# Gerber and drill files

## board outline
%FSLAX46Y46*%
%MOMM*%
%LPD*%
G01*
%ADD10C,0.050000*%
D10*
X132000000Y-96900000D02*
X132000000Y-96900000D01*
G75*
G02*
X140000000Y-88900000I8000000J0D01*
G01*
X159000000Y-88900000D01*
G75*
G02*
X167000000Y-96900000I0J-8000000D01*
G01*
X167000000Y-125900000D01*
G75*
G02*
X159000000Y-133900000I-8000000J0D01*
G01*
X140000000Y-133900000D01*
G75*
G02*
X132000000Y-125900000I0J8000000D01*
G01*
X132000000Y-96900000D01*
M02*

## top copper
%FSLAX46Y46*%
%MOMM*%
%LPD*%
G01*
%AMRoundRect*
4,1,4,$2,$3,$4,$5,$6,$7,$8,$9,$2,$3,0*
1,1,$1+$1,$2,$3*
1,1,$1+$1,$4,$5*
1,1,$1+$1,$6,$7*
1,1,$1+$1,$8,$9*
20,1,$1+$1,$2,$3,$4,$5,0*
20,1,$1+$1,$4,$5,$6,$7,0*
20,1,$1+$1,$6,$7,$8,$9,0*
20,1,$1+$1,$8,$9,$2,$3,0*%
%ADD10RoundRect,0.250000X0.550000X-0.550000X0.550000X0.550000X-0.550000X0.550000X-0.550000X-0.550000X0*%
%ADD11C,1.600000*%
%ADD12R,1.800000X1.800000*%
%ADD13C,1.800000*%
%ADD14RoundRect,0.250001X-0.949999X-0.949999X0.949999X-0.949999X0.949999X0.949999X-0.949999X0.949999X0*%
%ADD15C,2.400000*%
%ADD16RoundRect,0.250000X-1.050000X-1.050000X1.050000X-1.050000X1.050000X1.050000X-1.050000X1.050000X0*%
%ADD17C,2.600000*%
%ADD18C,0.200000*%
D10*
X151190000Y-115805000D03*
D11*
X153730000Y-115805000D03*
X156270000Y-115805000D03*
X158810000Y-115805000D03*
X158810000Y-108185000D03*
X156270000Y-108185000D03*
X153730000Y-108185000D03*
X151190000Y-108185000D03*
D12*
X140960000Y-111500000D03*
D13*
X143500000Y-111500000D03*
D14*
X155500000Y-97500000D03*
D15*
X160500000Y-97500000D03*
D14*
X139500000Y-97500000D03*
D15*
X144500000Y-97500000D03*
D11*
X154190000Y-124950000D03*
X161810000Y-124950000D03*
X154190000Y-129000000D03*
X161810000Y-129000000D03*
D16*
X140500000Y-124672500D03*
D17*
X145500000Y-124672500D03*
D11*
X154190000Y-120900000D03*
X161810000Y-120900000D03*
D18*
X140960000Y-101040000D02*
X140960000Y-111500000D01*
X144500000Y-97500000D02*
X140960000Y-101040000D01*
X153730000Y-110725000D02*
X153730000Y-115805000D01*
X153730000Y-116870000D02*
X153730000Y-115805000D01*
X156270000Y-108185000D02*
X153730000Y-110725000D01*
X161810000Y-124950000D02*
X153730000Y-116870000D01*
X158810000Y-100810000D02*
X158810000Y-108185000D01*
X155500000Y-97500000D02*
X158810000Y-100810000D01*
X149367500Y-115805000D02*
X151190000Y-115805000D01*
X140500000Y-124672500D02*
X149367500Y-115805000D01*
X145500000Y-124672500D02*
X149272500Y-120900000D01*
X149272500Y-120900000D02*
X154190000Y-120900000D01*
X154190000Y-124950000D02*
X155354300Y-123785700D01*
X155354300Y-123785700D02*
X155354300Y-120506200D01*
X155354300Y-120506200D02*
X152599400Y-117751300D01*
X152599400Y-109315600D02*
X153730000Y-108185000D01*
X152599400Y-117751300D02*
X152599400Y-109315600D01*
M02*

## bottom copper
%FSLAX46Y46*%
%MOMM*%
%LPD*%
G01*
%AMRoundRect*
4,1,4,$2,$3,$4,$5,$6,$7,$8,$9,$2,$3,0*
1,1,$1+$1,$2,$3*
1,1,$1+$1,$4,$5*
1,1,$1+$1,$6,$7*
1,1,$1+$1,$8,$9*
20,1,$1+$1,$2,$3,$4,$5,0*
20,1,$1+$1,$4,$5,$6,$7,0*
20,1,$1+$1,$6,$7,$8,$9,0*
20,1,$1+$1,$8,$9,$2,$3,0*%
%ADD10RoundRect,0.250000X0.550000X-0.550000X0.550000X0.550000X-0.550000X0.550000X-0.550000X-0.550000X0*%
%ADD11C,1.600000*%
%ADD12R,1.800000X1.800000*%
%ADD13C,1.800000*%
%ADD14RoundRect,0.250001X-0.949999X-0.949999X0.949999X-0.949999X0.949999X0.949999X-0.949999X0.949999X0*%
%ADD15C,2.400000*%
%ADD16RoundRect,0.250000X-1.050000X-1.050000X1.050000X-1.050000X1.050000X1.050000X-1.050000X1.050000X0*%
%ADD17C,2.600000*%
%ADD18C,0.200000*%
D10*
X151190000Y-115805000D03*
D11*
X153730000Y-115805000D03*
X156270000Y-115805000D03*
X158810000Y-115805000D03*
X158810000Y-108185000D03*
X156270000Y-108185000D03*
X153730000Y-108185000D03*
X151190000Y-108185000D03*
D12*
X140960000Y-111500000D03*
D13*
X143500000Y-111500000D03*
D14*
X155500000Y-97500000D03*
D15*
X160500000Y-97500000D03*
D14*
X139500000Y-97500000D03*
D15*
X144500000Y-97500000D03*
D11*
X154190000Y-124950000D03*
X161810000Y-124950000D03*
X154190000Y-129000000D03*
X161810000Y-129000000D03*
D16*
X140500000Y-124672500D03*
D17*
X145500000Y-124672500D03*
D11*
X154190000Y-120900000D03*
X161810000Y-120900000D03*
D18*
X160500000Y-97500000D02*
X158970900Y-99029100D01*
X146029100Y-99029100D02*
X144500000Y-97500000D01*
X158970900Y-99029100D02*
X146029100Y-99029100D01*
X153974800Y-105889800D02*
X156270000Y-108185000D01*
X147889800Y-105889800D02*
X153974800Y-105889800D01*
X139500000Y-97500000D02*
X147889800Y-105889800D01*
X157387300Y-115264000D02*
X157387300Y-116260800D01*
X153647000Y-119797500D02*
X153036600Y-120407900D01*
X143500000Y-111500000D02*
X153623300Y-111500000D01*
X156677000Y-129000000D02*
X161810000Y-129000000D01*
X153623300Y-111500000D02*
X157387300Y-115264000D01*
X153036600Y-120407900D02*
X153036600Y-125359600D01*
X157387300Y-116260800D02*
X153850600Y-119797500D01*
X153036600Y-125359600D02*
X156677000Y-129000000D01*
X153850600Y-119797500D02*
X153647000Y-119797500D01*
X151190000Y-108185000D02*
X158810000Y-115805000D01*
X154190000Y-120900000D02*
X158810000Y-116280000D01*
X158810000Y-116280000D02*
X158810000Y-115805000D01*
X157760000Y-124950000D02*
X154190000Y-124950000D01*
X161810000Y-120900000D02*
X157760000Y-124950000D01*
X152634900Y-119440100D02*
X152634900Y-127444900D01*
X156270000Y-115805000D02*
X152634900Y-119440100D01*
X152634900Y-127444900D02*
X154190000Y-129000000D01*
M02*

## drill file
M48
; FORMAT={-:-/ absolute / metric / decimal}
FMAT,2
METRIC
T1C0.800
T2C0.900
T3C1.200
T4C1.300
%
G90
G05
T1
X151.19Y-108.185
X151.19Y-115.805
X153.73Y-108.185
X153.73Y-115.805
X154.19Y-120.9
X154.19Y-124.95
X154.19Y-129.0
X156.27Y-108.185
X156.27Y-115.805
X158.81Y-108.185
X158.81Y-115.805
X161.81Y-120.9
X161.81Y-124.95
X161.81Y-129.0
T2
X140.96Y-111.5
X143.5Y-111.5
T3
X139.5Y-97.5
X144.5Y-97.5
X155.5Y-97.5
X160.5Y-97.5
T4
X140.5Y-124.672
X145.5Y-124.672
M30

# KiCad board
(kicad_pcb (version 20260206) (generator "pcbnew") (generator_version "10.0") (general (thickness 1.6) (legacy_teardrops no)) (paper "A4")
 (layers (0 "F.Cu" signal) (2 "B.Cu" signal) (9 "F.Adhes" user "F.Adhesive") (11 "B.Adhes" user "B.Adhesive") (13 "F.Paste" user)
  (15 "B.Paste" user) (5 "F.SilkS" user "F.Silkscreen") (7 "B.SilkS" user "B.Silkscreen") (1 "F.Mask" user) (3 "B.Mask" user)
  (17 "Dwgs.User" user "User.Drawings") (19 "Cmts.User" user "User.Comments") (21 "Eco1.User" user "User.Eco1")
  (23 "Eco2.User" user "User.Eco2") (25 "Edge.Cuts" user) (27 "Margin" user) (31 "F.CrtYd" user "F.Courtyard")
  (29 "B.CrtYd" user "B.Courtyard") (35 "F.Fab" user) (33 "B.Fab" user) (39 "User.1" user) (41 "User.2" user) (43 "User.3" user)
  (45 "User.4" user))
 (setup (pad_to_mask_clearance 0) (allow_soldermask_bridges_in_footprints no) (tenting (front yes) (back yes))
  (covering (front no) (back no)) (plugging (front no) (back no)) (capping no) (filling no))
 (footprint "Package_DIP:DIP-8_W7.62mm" (layer "F.Cu") (at 151.19 115.805 90)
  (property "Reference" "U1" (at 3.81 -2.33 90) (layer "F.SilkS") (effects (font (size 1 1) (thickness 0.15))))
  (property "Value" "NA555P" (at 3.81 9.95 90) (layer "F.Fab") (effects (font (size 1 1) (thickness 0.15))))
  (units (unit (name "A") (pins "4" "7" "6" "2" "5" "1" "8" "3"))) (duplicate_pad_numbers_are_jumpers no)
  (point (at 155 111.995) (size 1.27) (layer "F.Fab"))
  (pad "1" thru_hole roundrect (at 0 0 90) (size 1.6 1.6) (drill 0.8) (layers "*.Cu" "*.Mask") (remove_unused_layers no)
   (roundrect_rratio 0.15625) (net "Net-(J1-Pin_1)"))
  (pad "2" thru_hole circle (at 0 2.54 90) (size 1.6 1.6) (drill 0.8) (layers "*.Cu" "*.Mask") (remove_unused_layers no)
   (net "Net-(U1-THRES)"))
  (pad "3" thru_hole circle (at 0 5.08 90) (size 1.6 1.6) (drill 0.8) (layers "*.Cu" "*.Mask") (remove_unused_layers no)
   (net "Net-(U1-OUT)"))
  (pad "4" thru_hole circle (at 0 7.62 90) (size 1.6 1.6) (drill 0.8) (layers "*.Cu" "*.Mask") (remove_unused_layers no)
   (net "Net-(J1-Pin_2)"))
  (pad "5" thru_hole circle (at 7.62 7.62 90) (size 1.6 1.6) (drill 0.8) (layers "*.Cu" "*.Mask") (remove_unused_layers no)
   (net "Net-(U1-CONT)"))
  (pad "6" thru_hole circle (at 7.62 5.08 90) (size 1.6 1.6) (drill 0.8) (layers "*.Cu" "*.Mask") (remove_unused_layers no)
   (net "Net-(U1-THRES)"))
  (pad "7" thru_hole circle (at 7.62 2.54 90) (size 1.6 1.6) (drill 0.8) (layers "*.Cu" "*.Mask") (remove_unused_layers no)
   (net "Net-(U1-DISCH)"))
  (pad "8" thru_hole circle (at 7.62 0 90) (size 1.6 1.6) (drill 0.8) (layers "*.Cu" "*.Mask") (remove_unused_layers no)
   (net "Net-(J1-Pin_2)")))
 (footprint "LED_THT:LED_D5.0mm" (layer "F.Cu") (at 140.96 111.5)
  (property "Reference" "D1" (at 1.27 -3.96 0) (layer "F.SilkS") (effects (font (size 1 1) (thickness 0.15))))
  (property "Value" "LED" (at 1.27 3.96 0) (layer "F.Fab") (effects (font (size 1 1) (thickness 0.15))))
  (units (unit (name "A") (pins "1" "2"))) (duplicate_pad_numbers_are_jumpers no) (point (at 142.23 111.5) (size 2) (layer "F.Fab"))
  (pad "1" thru_hole rect (at 0 0) (size 1.8 1.8) (drill 0.9) (layers "*.Cu" "*.Mask") (remove_unused_layers no) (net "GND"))
  (pad "2" thru_hole circle (at 2.54 0) (size 1.8 1.8) (drill 0.9) (layers "*.Cu" "*.Mask") (remove_unused_layers no) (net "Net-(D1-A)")))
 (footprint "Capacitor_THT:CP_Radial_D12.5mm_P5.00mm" (layer "F.Cu") (at 155.5 97.5)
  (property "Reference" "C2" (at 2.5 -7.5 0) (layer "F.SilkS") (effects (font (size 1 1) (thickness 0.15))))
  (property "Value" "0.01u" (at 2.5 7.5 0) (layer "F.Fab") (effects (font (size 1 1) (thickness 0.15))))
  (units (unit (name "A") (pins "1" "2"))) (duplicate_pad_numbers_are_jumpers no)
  (pad "1" thru_hole roundrect (at 0 0) (size 2.4 2.4) (drill 1.2) (layers "*.Cu" "*.Mask") (remove_unused_layers no)
   (roundrect_rratio 0.104167) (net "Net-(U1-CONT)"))
  (pad "2" thru_hole circle (at 5 0) (size 2.4 2.4) (drill 1.2) (layers "*.Cu" "*.Mask") (remove_unused_layers no) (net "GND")))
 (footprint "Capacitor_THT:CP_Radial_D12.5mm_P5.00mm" (layer "F.Cu") (at 139.5 97.5)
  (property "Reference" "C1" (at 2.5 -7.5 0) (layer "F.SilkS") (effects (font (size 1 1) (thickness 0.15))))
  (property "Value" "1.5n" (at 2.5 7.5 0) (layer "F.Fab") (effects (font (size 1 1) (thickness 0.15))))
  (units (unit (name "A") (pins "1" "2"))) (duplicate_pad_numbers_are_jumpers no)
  (pad "1" thru_hole roundrect (at 0 0) (size 2.4 2.4) (drill 1.2) (layers "*.Cu" "*.Mask") (remove_unused_layers no)
   (roundrect_rratio 0.104167) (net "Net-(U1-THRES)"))
  (pad "2" thru_hole circle (at 5 0) (size 2.4 2.4) (drill 1.2) (layers "*.Cu" "*.Mask") (remove_unused_layers no) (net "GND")))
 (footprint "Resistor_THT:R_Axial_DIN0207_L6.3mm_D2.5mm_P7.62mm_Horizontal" (layer "F.Cu") (at 154.19 124.95)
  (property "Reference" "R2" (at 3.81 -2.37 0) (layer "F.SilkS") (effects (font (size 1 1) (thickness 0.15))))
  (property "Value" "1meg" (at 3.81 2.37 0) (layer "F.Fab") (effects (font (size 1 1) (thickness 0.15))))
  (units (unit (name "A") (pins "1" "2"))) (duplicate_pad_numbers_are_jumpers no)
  (pad "1" thru_hole circle (at 0 0) (size 1.6 1.6) (drill 0.8) (layers "*.Cu" "*.Mask") (remove_unused_layers no) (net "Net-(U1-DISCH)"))
  (pad "2" thru_hole circle (at 7.62 0) (size 1.6 1.6) (drill 0.8) (layers "*.Cu" "*.Mask") (remove_unused_layers no) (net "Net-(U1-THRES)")))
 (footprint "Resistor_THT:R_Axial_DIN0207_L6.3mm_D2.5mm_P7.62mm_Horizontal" (layer "F.Cu") (at 154.19 129)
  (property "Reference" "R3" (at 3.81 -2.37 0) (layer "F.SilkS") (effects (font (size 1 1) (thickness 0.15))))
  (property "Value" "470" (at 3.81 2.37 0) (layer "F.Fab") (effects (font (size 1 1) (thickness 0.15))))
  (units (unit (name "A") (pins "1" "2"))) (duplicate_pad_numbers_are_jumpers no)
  (pad "1" thru_hole circle (at 0 0) (size 1.6 1.6) (drill 0.8) (layers "*.Cu" "*.Mask") (remove_unused_layers no) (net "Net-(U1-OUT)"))
  (pad "2" thru_hole circle (at 7.62 0) (size 1.6 1.6) (drill 0.8) (layers "*.Cu" "*.Mask") (remove_unused_layers no) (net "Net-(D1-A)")))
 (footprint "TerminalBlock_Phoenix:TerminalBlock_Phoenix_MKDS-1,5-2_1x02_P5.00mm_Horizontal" (layer "F.Cu") (at 140.5 124.6725)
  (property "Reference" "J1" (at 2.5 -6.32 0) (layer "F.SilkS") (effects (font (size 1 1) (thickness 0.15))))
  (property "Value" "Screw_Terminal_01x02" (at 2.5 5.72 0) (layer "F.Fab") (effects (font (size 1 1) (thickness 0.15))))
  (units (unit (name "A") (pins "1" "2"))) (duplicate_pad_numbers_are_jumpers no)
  (pad "1" thru_hole roundrect (at 0 0) (size 2.6 2.6) (drill 1.3) (layers "*.Cu" "*.Mask") (remove_unused_layers no)
   (roundrect_rratio 0.096154) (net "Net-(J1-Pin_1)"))
  (pad "2" thru_hole circle (at 5 0) (size 2.6 2.6) (drill 1.3) (layers "*.Cu" "*.Mask") (remove_unused_layers no) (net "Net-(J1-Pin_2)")))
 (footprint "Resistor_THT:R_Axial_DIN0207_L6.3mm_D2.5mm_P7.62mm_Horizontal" (layer "F.Cu") (at 154.19 120.9)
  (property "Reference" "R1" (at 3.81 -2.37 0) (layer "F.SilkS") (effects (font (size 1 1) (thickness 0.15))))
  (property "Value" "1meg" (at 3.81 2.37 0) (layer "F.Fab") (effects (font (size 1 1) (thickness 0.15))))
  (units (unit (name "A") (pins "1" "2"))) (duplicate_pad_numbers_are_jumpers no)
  (pad "1" thru_hole circle (at 0 0) (size 1.6 1.6) (drill 0.8) (layers "*.Cu" "*.Mask") (remove_unused_layers no) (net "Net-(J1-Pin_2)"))
  (pad "2" thru_hole circle (at 7.62 0) (size 1.6 1.6) (drill 0.8) (layers "*.Cu" "*.Mask") (remove_unused_layers no) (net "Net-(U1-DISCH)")))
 (gr_rect (start 132 88.9) (end 167 133.9) (radius 8) (stroke (width 0.05) (type solid)) (fill no) (layer "Edge.Cuts"))
 (segment (start 140.96 101.04) (end 140.96 111.5) (width 0.2) (layer "F.Cu") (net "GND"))
 (segment (start 144.5 97.5) (end 140.96 101.04) (width 0.2) (layer "F.Cu") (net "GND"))
 (segment (start 160.5 97.5) (end 158.9709 99.0291) (width 0.2) (layer "B.Cu") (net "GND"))
 (segment (start 146.0291 99.0291) (end 144.5 97.5) (width 0.2) (layer "B.Cu") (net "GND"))
 (segment (start 158.9709 99.0291) (end 146.0291 99.0291) (width 0.2) (layer "B.Cu") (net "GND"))
 (segment (start 153.73 110.725) (end 153.73 115.805) (width 0.2) (layer "F.Cu") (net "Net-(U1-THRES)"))
 (segment (start 153.73 116.87) (end 153.73 115.805) (width 0.2) (layer "F.Cu") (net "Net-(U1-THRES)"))
 (segment (start 156.27 108.185) (end 153.73 110.725) (width 0.2) (layer "F.Cu") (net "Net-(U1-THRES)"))
 (segment (start 161.81 124.95) (end 153.73 116.87) (width 0.2) (layer "F.Cu") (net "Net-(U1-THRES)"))
 (segment (start 153.9748 105.8898) (end 156.27 108.185) (width 0.2) (layer "B.Cu") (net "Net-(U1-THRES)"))
 (segment (start 147.8898 105.8898) (end 153.9748 105.8898) (width 0.2) (layer "B.Cu") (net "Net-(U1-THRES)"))
 (segment (start 139.5 97.5) (end 147.8898 105.8898) (width 0.2) (layer "B.Cu") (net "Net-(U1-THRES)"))
 (segment (start 158.81 100.81) (end 158.81 108.185) (width 0.2) (layer "F.Cu") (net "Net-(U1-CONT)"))
 (segment (start 155.5 97.5) (end 158.81 100.81) (width 0.2) (layer "F.Cu") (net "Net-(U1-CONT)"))
 (segment (start 157.3873 115.264) (end 157.3873 116.2608) (width 0.2) (layer "B.Cu") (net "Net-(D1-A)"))
 (segment (start 153.647 119.7975) (end 153.0366 120.4079) (width 0.2) (layer "B.Cu") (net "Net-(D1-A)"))
 (segment (start 143.5 111.5) (end 153.6233 111.5) (width 0.2) (layer "B.Cu") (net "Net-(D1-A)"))
 (segment (start 156.677 129) (end 161.81 129) (width 0.2) (layer "B.Cu") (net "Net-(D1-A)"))
 (segment (start 153.6233 111.5) (end 157.3873 115.264) (width 0.2) (layer "B.Cu") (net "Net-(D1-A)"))
 (segment (start 153.0366 120.4079) (end 153.0366 125.3596) (width 0.2) (layer "B.Cu") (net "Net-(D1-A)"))
 (segment (start 157.3873 116.2608) (end 153.8506 119.7975) (width 0.2) (layer "B.Cu") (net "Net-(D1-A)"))
 (segment (start 153.0366 125.3596) (end 156.677 129) (width 0.2) (layer "B.Cu") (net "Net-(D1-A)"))
 (segment (start 153.8506 119.7975) (end 153.647 119.7975) (width 0.2) (layer "B.Cu") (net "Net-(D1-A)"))
 (segment (start 149.3675 115.805) (end 151.19 115.805) (width 0.2) (layer "F.Cu") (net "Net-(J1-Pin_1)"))
 (segment (start 140.5 124.6725) (end 149.3675 115.805) (width 0.2) (layer "F.Cu") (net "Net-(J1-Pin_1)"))
 (segment (start 145.5 124.6725) (end 149.2725 120.9) (width 0.2) (layer "F.Cu") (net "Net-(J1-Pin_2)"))
 (segment (start 149.2725 120.9) (end 154.19 120.9) (width 0.2) (layer "F.Cu") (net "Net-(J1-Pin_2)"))
 (segment (start 151.19 108.185) (end 158.81 115.805) (width 0.2) (layer "B.Cu") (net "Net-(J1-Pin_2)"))
 (segment (start 154.19 120.9) (end 158.81 116.28) (width 0.2) (layer "B.Cu") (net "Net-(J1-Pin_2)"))
 (segment (start 158.81 116.28) (end 158.81 115.805) (width 0.2) (layer "B.Cu") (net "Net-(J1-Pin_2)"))
 (segment (start 154.19 124.95) (end 155.3543 123.7857) (width 0.2) (layer "F.Cu") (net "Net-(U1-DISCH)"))
 (segment (start 155.3543 123.7857) (end 155.3543 120.5062) (width 0.2) (layer "F.Cu") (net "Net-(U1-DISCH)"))
 (segment (start 155.3543 120.5062) (end 152.5994 117.7513) (width 0.2) (layer "F.Cu") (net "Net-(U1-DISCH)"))
 (segment (start 152.5994 109.3156) (end 153.73 108.185) (width 0.2) (layer "F.Cu") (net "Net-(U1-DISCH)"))
 (segment (start 152.5994 117.7513) (end 152.5994 109.3156) (width 0.2) (layer "F.Cu") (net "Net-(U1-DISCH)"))
 (segment (start 157.76 124.95) (end 154.19 124.95) (width 0.2) (layer "B.Cu") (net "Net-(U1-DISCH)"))
 (segment (start 161.81 120.9) (end 157.76 124.95) (width 0.2) (layer "B.Cu") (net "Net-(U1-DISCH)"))
 (segment (start 152.6349 119.4401) (end 152.6349 127.4449) (width 0.2) (layer "B.Cu") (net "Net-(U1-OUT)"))
 (segment (start 156.27 115.805) (end 152.6349 119.4401) (width 0.2) (layer "B.Cu") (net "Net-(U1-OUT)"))
 (segment (start 152.6349 127.4449) (end 154.19 129) (width 0.2) (layer "B.Cu") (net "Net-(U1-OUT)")))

